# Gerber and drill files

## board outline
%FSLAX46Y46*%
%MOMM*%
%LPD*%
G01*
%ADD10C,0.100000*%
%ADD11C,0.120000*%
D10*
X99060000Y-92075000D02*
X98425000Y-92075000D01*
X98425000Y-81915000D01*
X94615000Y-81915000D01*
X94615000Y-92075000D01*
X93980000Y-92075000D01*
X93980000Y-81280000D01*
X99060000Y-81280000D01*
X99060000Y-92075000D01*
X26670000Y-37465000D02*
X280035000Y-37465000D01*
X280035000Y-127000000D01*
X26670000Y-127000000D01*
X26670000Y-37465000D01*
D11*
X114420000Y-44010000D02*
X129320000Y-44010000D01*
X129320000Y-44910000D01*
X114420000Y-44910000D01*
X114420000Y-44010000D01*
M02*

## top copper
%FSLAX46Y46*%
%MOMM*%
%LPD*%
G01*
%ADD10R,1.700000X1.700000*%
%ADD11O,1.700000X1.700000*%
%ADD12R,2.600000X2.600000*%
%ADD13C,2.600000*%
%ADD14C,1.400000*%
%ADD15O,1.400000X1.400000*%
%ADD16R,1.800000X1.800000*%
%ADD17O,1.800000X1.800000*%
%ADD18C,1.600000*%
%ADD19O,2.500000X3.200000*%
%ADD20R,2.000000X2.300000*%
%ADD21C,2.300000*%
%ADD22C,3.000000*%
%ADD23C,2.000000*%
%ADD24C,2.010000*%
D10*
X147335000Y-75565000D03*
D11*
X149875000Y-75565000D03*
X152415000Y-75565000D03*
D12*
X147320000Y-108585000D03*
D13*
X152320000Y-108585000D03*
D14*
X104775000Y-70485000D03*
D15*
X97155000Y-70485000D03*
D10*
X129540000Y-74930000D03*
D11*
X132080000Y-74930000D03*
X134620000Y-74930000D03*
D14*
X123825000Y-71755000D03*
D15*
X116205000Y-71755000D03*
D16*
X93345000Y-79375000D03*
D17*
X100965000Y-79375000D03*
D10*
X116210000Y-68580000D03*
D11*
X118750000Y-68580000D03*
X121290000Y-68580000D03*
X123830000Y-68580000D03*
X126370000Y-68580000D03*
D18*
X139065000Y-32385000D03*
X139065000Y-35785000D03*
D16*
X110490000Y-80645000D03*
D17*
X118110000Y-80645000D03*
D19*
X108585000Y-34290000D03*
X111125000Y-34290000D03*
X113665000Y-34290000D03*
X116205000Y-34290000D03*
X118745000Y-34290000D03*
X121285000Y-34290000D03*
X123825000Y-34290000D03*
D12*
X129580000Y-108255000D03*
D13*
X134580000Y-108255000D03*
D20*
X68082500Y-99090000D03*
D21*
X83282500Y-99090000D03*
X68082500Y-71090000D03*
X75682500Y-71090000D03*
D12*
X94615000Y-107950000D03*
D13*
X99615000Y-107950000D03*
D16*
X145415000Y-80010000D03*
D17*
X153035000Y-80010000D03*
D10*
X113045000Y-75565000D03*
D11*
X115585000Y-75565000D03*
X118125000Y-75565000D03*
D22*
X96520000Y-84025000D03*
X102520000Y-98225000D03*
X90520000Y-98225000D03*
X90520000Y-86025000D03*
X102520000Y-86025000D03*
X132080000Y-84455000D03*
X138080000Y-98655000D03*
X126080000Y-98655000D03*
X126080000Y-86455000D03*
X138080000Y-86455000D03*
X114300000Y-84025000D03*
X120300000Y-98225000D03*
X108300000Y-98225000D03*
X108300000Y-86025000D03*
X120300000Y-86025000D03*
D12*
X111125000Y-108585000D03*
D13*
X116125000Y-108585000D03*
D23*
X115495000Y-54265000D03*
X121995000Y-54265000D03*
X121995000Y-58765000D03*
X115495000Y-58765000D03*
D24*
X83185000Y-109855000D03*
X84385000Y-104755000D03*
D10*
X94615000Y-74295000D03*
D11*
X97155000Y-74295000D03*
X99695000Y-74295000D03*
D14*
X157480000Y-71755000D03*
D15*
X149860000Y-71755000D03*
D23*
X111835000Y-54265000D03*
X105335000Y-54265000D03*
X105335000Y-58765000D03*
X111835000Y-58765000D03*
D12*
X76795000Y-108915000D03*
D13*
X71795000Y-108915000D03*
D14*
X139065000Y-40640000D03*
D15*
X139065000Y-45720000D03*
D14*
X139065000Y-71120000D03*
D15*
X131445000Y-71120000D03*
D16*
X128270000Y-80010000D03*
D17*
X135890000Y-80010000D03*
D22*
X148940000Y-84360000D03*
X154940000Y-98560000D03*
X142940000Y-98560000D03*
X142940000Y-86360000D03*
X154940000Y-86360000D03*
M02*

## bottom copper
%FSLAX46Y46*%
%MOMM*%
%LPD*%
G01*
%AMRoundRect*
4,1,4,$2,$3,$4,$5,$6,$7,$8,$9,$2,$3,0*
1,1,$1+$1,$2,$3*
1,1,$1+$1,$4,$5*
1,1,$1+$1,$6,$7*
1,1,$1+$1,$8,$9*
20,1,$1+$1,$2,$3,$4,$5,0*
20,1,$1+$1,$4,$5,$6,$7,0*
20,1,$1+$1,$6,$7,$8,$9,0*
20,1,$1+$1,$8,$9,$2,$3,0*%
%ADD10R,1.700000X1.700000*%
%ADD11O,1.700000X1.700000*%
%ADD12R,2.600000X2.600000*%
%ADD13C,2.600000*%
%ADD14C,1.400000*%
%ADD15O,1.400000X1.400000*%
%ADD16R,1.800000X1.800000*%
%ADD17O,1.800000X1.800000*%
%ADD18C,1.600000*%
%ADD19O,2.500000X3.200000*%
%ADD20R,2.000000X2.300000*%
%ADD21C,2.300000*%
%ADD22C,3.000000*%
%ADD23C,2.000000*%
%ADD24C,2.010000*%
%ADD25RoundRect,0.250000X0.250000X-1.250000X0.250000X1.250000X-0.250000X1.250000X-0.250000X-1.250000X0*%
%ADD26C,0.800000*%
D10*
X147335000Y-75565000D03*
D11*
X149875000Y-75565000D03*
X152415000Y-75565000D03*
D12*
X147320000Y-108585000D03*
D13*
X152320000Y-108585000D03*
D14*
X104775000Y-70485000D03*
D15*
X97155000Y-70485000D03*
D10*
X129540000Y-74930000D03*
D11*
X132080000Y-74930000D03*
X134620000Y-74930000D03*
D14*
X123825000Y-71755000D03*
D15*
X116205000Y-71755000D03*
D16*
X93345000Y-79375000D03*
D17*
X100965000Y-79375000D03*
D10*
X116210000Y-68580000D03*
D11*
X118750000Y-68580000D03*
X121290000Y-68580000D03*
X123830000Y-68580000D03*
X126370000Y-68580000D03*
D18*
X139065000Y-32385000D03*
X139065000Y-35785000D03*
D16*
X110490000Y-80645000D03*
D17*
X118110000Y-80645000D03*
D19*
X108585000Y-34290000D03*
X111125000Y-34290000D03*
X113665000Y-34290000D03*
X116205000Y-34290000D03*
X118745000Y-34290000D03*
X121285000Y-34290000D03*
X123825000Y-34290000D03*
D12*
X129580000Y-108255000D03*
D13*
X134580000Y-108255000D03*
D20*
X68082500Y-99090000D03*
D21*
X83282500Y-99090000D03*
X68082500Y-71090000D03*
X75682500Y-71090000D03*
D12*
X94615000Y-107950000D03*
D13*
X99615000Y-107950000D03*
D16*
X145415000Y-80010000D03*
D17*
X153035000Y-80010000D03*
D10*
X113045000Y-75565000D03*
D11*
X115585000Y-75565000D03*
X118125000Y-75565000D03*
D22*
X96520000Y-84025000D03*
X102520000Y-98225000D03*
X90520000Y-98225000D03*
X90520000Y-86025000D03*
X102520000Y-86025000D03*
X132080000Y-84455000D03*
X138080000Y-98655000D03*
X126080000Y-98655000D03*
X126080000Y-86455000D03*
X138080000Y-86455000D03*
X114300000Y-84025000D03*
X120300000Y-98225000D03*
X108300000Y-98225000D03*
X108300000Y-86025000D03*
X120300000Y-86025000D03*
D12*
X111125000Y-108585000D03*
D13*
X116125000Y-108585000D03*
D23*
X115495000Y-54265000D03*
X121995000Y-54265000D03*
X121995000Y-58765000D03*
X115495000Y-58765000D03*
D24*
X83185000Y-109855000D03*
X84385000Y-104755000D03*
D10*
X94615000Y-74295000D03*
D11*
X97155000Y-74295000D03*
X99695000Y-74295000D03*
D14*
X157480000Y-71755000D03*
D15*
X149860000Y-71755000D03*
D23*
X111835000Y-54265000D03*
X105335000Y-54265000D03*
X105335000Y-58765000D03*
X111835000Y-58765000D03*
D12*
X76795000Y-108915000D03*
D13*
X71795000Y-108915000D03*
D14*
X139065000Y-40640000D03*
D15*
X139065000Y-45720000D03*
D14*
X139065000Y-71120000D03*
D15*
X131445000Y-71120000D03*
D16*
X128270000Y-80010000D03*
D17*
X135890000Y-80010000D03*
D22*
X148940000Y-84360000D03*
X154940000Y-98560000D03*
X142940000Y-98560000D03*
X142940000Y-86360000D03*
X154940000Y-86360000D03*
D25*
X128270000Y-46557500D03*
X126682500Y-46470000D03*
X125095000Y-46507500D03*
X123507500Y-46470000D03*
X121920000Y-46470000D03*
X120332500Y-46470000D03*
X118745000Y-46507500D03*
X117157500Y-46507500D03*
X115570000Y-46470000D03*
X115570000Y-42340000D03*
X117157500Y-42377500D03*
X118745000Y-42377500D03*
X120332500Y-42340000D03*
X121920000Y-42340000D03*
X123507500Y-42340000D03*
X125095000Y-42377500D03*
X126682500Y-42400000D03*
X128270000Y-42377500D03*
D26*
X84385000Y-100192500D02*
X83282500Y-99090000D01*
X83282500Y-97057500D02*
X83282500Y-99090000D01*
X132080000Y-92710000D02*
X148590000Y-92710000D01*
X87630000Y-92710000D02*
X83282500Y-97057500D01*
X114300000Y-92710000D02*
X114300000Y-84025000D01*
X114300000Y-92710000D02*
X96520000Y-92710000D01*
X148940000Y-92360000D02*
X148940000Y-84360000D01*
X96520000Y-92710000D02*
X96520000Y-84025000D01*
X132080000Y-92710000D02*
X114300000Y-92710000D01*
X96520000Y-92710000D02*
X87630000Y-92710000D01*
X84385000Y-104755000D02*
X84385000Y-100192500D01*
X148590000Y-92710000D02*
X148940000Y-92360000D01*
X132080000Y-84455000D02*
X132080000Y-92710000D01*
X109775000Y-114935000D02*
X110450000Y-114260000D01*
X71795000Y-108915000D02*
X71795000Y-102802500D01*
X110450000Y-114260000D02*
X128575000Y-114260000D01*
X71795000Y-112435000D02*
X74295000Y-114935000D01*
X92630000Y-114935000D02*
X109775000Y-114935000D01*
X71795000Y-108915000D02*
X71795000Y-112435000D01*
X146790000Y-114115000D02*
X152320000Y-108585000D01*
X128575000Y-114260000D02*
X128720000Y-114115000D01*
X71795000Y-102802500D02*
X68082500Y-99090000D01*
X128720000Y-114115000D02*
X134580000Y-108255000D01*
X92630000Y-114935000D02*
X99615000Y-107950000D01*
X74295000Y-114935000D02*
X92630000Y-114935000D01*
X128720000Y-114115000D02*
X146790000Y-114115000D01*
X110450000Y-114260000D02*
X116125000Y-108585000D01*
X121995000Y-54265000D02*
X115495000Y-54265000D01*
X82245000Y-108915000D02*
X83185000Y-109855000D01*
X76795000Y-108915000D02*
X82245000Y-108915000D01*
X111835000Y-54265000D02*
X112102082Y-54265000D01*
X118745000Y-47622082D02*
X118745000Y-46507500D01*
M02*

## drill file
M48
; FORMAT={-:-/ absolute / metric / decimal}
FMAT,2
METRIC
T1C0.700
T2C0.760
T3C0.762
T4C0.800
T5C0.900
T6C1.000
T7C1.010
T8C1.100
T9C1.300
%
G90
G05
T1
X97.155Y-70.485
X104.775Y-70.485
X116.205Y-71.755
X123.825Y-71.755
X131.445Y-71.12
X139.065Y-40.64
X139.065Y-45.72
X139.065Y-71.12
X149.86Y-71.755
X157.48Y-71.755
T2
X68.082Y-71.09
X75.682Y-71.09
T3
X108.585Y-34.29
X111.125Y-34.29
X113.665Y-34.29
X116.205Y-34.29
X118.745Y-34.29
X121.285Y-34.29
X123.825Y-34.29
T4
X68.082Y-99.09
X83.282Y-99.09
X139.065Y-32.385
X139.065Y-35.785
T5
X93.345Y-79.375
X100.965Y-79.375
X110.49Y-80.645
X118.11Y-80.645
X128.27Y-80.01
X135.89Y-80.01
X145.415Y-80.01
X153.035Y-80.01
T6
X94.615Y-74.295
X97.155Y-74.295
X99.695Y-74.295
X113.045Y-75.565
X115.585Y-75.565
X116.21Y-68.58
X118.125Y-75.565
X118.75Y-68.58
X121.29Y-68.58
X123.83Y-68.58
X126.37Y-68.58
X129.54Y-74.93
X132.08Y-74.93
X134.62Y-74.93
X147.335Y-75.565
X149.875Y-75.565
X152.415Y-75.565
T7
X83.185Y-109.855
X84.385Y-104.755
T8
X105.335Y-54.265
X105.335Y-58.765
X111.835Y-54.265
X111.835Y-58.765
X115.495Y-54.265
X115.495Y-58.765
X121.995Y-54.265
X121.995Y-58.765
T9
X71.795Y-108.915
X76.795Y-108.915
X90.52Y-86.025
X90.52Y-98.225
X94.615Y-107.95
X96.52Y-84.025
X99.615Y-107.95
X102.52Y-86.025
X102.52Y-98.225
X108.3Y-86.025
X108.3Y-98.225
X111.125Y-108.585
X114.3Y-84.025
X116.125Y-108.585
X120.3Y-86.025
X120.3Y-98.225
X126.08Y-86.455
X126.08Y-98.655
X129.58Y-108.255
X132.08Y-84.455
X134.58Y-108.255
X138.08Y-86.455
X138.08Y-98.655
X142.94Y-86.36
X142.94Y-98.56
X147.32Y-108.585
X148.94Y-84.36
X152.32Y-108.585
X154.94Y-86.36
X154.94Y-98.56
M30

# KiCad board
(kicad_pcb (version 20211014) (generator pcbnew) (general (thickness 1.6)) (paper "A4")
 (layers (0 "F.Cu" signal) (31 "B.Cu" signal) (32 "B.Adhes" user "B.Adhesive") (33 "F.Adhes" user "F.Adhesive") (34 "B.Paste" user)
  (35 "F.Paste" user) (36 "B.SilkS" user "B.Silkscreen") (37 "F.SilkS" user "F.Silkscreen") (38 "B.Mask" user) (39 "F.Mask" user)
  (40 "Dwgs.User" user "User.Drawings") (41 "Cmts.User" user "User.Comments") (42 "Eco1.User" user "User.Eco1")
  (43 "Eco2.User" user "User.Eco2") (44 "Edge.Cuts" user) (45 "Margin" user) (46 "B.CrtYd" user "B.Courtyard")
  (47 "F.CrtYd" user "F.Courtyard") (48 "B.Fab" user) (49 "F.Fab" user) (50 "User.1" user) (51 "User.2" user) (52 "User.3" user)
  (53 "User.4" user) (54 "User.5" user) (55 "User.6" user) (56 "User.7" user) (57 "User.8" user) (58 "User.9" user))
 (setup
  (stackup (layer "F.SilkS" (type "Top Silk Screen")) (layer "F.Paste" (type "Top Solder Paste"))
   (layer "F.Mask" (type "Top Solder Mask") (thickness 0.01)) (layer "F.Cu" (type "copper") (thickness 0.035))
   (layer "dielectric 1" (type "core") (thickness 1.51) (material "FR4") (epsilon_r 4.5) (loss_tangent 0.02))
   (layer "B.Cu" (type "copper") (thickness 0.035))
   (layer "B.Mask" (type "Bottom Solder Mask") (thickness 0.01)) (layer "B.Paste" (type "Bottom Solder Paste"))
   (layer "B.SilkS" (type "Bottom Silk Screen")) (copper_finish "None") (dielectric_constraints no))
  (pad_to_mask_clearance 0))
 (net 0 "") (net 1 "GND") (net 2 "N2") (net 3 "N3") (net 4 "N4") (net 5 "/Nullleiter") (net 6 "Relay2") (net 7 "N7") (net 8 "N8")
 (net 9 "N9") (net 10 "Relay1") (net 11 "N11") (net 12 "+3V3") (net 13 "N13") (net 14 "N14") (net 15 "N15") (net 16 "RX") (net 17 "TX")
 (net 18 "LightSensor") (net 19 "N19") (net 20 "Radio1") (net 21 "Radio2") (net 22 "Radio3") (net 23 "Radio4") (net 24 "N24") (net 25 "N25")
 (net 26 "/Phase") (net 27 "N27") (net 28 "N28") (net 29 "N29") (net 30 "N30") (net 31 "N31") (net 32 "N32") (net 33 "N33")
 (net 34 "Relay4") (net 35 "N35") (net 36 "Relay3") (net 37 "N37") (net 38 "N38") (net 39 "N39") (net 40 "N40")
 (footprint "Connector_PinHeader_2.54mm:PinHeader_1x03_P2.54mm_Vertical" (layer "F.Cu") (at 147.335 75.565 90)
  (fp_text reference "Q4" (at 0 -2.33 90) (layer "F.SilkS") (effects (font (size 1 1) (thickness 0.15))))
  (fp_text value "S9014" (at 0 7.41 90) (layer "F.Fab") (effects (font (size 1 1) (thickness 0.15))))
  (pad "1" thru_hole rect (at 0 0 90) (size 1.7 1.7) (drill 1) (layers *.Cu *.Mask) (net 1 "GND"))
  (pad "2" thru_hole oval (at 0 2.54 90) (size 1.7 1.7) (drill 1) (layers *.Cu *.Mask) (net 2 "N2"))
  (pad "3" thru_hole oval (at 0 5.08 90) (size 1.7 1.7) (drill 1) (layers *.Cu *.Mask) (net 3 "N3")))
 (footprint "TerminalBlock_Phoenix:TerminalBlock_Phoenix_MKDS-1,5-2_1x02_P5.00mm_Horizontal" (layer "F.Cu") (at 147.32 108.585)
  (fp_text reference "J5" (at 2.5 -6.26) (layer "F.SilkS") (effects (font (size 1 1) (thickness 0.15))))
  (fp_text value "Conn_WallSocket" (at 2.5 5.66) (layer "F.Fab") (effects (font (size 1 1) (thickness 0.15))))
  (pad "1" thru_hole rect (at 0 0) (size 2.6 2.6) (drill 1.3) (layers *.Cu *.Mask) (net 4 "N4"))
  (pad "2" thru_hole circle (at 5 0) (size 2.6 2.6) (drill 1.3) (layers *.Cu *.Mask) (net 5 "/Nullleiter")))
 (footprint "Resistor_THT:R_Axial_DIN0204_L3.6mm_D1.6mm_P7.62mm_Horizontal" (layer "F.Cu") (at 104.775 70.485 180)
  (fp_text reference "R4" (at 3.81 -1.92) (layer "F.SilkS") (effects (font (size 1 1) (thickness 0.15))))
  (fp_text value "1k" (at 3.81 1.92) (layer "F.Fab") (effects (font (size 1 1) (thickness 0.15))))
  (pad "1" thru_hole circle (at 0 0 180) (size 1.4 1.4) (drill 0.7) (layers *.Cu *.Mask) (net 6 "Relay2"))
  (pad "2" thru_hole oval (at 7.62 0 180) (size 1.4 1.4) (drill 0.7) (layers *.Cu *.Mask) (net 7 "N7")))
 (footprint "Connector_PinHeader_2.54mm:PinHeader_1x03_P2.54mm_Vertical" (layer "F.Cu") (at 129.54 74.93 90)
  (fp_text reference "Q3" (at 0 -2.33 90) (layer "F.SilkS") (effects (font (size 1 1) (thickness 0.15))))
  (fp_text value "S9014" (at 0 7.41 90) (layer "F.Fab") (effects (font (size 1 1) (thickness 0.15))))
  (pad "1" thru_hole rect (at 0 0 90) (size 1.7 1.7) (drill 1) (layers *.Cu *.Mask) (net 1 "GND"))
  (pad "2" thru_hole oval (at 0 2.54 90) (size 1.7 1.7) (drill 1) (layers *.Cu *.Mask) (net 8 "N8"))
  (pad "3" thru_hole oval (at 0 5.08 90) (size 1.7 1.7) (drill 1) (layers *.Cu *.Mask) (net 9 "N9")))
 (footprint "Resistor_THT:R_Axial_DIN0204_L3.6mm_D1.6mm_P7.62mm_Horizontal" (layer "F.Cu") (at 123.825 71.755 180)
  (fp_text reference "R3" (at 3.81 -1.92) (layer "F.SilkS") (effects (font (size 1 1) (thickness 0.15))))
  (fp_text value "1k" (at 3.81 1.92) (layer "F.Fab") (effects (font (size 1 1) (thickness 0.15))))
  (pad "1" thru_hole circle (at 0 0 180) (size 1.4 1.4) (drill 0.7) (layers *.Cu *.Mask) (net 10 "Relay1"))
  (pad "2" thru_hole oval (at 7.62 0 180) (size 1.4 1.4) (drill 0.7) (layers *.Cu *.Mask) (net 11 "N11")))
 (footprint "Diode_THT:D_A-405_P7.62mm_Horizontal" (layer "F.Cu") (at 93.345 79.375)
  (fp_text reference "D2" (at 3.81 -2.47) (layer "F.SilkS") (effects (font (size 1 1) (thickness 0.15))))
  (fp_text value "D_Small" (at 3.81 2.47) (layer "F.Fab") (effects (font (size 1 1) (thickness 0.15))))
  (pad "1" thru_hole rect (at 0 0) (size 1.8 1.8) (drill 0.9) (layers *.Cu *.Mask) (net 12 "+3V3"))
  (pad "2" thru_hole oval (at 7.62 0) (size 1.8 1.8) (drill 0.9) (layers *.Cu *.Mask) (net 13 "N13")))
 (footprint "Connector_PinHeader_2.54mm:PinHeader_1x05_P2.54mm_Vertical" (layer "F.Cu") (at 116.21 68.58 90)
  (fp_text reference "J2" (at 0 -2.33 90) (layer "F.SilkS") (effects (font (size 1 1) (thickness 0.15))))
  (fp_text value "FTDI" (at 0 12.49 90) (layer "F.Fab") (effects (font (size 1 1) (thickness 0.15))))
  (pad "1" thru_hole rect (at 0 0 90) (size 1.7 1.7) (drill 1) (layers *.Cu *.Mask) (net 1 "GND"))
  (pad "2" thru_hole oval (at 0 2.54 90) (size 1.7 1.7) (drill 1) (layers *.Cu *.Mask) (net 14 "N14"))
  (pad "3" thru_hole oval (at 0 5.08 90) (size 1.7 1.7) (drill 1) (layers *.Cu *.Mask) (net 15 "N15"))
  (pad "4" thru_hole oval (at 0 7.62 90) (size 1.7 1.7) (drill 1) (layers *.Cu *.Mask) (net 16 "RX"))
  (pad "5" thru_hole oval (at 0 10.16 90) (size 1.7 1.7) (drill 1) (layers *.Cu *.Mask) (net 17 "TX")))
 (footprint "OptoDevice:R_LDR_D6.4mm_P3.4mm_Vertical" (layer "F.Cu") (at 139.065 32.385 -90)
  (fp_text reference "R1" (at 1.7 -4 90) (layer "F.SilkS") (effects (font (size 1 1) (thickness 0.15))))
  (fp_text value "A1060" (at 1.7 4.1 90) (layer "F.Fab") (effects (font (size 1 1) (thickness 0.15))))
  (pad "1" thru_hole circle (at 0 0 270) (size 1.6 1.6) (drill 0.8) (layers *.Cu *.Mask) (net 12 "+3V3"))
  (pad "2" thru_hole circle (at 3.4 0 270) (size 1.6 1.6) (drill 0.8) (layers *.Cu *.Mask) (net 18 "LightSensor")))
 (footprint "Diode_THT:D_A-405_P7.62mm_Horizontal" (layer "F.Cu") (at 110.49 80.645)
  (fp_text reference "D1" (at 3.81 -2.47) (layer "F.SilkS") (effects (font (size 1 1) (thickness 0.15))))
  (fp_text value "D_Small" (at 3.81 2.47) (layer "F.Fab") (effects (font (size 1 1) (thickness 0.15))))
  (pad "1" thru_hole rect (at 0 0) (size 1.8 1.8) (drill 0.9) (layers *.Cu *.Mask) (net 12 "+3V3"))
  (pad "2" thru_hole oval (at 7.62 0) (size 1.8 1.8) (drill 0.9) (layers *.Cu *.Mask) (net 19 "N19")))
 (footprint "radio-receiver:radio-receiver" (layer "F.Cu") (at 108.585 34.29)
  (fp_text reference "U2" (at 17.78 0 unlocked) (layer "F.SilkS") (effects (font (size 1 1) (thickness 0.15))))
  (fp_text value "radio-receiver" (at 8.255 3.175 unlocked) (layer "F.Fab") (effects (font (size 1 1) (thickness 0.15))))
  (pad "1" thru_hole oval (at 0 0 270) (size 3.2 2.5) (drill 0.762) (layers *.Cu *.Mask) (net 1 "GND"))
  (pad "2" thru_hole oval (at 2.54 0 270) (size 3.2 2.5) (drill 0.762) (layers *.Cu *.Mask) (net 12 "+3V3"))
  (pad "3" thru_hole oval (at 5.08 0 270) (size 3.2 2.5) (drill 0.762) (layers *.Cu *.Mask) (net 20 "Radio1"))
  (pad "4" thru_hole oval (at 7.62 0 270) (size 3.2 2.5) (drill 0.762) (layers *.Cu *.Mask) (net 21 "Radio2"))
  (pad "5" thru_hole oval (at 10.16 0 270) (size 3.2 2.5) (drill 0.762) (layers *.Cu *.Mask) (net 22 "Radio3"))
  (pad "6" thru_hole oval (at 12.7 0 270) (size 3.2 2.5) (drill 0.762) (layers *.Cu *.Mask) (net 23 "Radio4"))
  (pad "7" thru_hole oval (at 15.24 0 270) (size 3.2 2.5) (drill 0.762) (layers *.Cu *.Mask) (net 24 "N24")))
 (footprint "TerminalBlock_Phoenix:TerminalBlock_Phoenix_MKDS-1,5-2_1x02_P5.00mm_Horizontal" (layer "F.Cu") (at 129.58 108.255)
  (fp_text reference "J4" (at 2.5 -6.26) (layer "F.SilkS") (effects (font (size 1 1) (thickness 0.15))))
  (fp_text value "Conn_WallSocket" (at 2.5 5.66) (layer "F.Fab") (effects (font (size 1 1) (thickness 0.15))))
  (pad "1" thru_hole rect (at 0 0) (size 2.6 2.6) (drill 1.3) (layers *.Cu *.Mask) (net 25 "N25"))
  (pad "2" thru_hole circle (at 5 0) (size 2.6 2.6) (drill 1.3) (layers *.Cu *.Mask) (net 5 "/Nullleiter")))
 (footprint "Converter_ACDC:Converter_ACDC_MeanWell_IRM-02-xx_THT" (layer "F.Cu") (at 68.0825 99.09 90)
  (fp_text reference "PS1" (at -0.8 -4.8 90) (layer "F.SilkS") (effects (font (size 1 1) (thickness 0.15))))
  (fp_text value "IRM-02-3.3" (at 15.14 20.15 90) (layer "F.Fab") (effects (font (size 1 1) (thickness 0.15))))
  (pad "1" thru_hole rect (at 0 0 90) (size 2.3 2) (drill 0.8) (layers *.Cu *.Mask) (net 5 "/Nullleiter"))
  (pad "2" thru_hole circle (at 0 15.2 90) (size 2.3 2.3) (drill 0.8) (layers *.Cu *.Mask) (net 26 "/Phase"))
  (pad "3" thru_hole circle (at 28 0 90) (size 2.3 2.3) (drill 0.76) (layers *.Cu *.Mask) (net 1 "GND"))
  (pad "4" thru_hole circle (at 28 7.6 90) (size 2.3 2.3) (drill 0.76) (layers *.Cu *.Mask) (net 12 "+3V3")))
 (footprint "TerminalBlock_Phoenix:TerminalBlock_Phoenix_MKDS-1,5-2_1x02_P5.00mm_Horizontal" (layer "F.Cu") (at 94.615 107.95)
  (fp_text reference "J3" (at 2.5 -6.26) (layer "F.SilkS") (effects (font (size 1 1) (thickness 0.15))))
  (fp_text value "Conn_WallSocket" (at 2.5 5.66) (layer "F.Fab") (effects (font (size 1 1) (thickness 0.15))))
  (pad "1" thru_hole rect (at 0 0) (size 2.6 2.6) (drill 1.3) (layers *.Cu *.Mask) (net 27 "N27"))
  (pad "2" thru_hole circle (at 5 0) (size 2.6 2.6) (drill 1.3) (layers *.Cu *.Mask) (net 5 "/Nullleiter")))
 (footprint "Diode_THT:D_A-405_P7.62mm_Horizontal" (layer "F.Cu") (at 145.415 80.01)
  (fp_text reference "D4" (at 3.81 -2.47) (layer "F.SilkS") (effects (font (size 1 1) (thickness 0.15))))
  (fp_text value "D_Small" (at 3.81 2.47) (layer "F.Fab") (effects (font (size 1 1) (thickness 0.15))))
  (pad "1" thru_hole rect (at 0 0) (size 1.8 1.8) (drill 0.9) (layers *.Cu *.Mask) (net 12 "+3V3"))
  (pad "2" thru_hole oval (at 7.62 0) (size 1.8 1.8) (drill 0.9) (layers *.Cu *.Mask) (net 3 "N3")))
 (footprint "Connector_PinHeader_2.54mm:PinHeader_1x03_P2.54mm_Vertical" (layer "F.Cu") (at 113.045 75.565 90)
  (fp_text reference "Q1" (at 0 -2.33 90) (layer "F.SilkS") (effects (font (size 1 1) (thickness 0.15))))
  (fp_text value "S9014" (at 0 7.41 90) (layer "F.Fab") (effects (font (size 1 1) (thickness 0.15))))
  (pad "1" thru_hole rect (at 0 0 90) (size 1.7 1.7) (drill 1) (layers *.Cu *.Mask) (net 1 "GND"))
  (pad "2" thru_hole oval (at 0 2.54 90) (size 1.7 1.7) (drill 1) (layers *.Cu *.Mask) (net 11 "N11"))
  (pad "3" thru_hole oval (at 0 5.08 90) (size 1.7 1.7) (drill 1) (layers *.Cu *.Mask) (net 19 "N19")))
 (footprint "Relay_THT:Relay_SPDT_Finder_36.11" (layer "F.Cu") (at 96.52 84.025 -90)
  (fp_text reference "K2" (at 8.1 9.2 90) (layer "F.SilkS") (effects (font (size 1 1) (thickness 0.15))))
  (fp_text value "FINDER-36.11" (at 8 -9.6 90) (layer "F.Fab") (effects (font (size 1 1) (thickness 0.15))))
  (pad "11" thru_hole circle (at 0 0 270) (size 3 3) (drill 1.3) (layers *.Cu *.Mask) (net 26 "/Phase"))
  (pad "12" thru_hole circle (at 14.2 -6 270) (size 3 3) (drill 1.3) (layers *.Cu *.Mask) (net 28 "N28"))
  (pad "14" thru_hole circle (at 14.2 6 270) (size 3 3) (drill 1.3) (layers *.Cu *.Mask) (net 27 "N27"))
  (pad "A1" thru_hole circle (at 2 6 270) (size 3 3) (drill 1.3) (layers *.Cu *.Mask) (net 12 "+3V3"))
  (pad "A2" thru_hole circle (at 2 -6 270) (size 3 3) (drill 1.3) (layers *.Cu *.Mask) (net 13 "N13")))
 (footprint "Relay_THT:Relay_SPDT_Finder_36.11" (layer "F.Cu") (at 132.08 84.455 -90)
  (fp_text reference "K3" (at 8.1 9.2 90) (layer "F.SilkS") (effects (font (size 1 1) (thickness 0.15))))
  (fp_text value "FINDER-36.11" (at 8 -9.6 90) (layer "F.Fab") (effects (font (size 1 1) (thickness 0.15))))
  (pad "11" thru_hole circle (at 0 0 270) (size 3 3) (drill 1.3) (layers *.Cu *.Mask) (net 26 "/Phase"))
  (pad "12" thru_hole circle (at 14.2 -6 270) (size 3 3) (drill 1.3) (layers *.Cu *.Mask) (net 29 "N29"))
  (pad "14" thru_hole circle (at 14.2 6 270) (size 3 3) (drill 1.3) (layers *.Cu *.Mask) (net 25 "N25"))
  (pad "A1" thru_hole circle (at 2 6 270) (size 3 3) (drill 1.3) (layers *.Cu *.Mask) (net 12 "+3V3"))
  (pad "A2" thru_hole circle (at 2 -6 270) (size 3 3) (drill 1.3) (layers *.Cu *.Mask) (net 9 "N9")))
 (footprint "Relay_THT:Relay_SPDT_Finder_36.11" (layer "F.Cu") (at 114.3 84.025 -90)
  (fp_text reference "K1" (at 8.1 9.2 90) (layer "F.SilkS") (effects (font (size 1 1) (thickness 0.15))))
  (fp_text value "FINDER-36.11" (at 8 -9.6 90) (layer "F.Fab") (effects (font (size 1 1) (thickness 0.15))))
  (pad "11" thru_hole circle (at 0 0 270) (size 3 3) (drill 1.3) (layers *.Cu *.Mask) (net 26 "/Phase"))
  (pad "12" thru_hole circle (at 14.2 -6 270) (size 3 3) (drill 1.3) (layers *.Cu *.Mask) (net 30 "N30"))
  (pad "14" thru_hole circle (at 14.2 6 270) (size 3 3) (drill 1.3) (layers *.Cu *.Mask) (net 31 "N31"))
  (pad "A1" thru_hole circle (at 2 6 270) (size 3 3) (drill 1.3) (layers *.Cu *.Mask) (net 12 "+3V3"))
  (pad "A2" thru_hole circle (at 2 -6 270) (size 3 3) (drill 1.3) (layers *.Cu *.Mask) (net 19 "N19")))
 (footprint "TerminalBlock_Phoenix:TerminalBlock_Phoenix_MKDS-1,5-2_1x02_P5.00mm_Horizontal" (layer "F.Cu") (at 111.125 108.585)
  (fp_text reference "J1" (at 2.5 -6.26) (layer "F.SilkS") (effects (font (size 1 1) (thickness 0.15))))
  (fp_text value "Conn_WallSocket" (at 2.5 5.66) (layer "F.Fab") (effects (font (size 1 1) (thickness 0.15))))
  (pad "1" thru_hole rect (at 0 0) (size 2.6 2.6) (drill 1.3) (layers *.Cu *.Mask) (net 31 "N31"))
  (pad "2" thru_hole circle (at 5 0) (size 2.6 2.6) (drill 1.3) (layers *.Cu *.Mask) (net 5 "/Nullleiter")))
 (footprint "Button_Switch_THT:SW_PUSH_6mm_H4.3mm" (layer "F.Cu") (at 115.495 54.265)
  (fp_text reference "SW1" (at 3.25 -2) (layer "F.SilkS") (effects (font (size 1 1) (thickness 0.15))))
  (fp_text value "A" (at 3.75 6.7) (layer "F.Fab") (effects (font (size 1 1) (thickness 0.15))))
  (pad "1" thru_hole circle (at 0 0 90) (size 2 2) (drill 1.1) (layers *.Cu *.Mask) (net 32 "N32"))
  (pad "1" thru_hole circle (at 6.5 0 90) (size 2 2) (drill 1.1) (layers *.Cu *.Mask) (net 32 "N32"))
  (pad "2" thru_hole circle (at 6.5 4.5 90) (size 2 2) (drill 1.1) (layers *.Cu *.Mask) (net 1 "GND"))
  (pad "2" thru_hole circle (at 0 4.5 90) (size 2 2) (drill 1.1) (layers *.Cu *.Mask) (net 1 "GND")))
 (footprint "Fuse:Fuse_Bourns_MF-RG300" (layer "F.Cu") (at 83.185 109.855 90)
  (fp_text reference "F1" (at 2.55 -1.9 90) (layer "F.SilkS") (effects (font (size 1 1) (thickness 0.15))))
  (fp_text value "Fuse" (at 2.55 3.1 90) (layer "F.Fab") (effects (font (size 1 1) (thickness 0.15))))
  (pad "1" thru_hole circle (at 0 0 90) (size 2.01 2.01) (drill 1.01) (layers *.Cu *.Mask) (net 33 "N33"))
  (pad "2" thru_hole circle (at 5.1 1.2 90) (size 2.01 2.01) (drill 1.01) (layers *.Cu *.Mask) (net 26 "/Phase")))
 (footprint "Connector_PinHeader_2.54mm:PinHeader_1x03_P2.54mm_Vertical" (layer "F.Cu") (at 94.615 74.295 90)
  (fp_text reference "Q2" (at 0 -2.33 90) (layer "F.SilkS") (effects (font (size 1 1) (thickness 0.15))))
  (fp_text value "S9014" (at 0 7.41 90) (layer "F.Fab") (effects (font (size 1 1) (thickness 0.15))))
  (pad "1" thru_hole rect (at 0 0 90) (size 1.7 1.7) (drill 1) (layers *.Cu *.Mask) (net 1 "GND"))
  (pad "2" thru_hole oval (at 0 2.54 90) (size 1.7 1.7) (drill 1) (layers *.Cu *.Mask) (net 7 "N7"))
  (pad "3" thru_hole oval (at 0 5.08 90) (size 1.7 1.7) (drill 1) (layers *.Cu *.Mask) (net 13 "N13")))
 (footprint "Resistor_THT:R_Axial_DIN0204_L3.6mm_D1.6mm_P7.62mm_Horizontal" (layer "F.Cu") (at 157.48 71.755 180)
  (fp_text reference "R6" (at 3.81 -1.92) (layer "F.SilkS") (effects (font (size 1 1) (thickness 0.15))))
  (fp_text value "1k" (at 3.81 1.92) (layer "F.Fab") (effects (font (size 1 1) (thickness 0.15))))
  (pad "1" thru_hole circle (at 0 0 180) (size 1.4 1.4) (drill 0.7) (layers *.Cu *.Mask) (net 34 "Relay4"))
  (pad "2" thru_hole oval (at 7.62 0 180) (size 1.4 1.4) (drill 0.7) (layers *.Cu *.Mask) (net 2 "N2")))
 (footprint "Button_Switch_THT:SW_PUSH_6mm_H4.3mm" (layer "F.Cu") (at 105.335 54.265)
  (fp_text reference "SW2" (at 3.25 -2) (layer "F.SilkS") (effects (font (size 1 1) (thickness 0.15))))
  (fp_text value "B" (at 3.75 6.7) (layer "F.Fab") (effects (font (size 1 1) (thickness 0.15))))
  (pad "1" thru_hole circle (at 6.5 0 90) (size 2 2) (drill 1.1) (layers *.Cu *.Mask) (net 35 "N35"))
  (pad "1" thru_hole circle (at 0 0 90) (size 2 2) (drill 1.1) (layers *.Cu *.Mask) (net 35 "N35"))
  (pad "2" thru_hole circle (at 0 4.5 90) (size 2 2) (drill 1.1) (layers *.Cu *.Mask) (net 1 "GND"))
  (pad "2" thru_hole circle (at 6.5 4.5 90) (size 2 2) (drill 1.1) (layers *.Cu *.Mask) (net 1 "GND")))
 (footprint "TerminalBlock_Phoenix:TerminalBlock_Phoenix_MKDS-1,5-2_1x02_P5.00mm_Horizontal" (layer "F.Cu") (at 76.795 108.915 180)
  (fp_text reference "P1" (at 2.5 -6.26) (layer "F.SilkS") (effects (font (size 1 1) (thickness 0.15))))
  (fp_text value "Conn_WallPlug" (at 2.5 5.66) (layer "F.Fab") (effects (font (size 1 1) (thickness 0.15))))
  (pad "1" thru_hole rect (at 0 0 180) (size 2.6 2.6) (drill 1.3) (layers *.Cu *.Mask) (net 33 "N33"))
  (pad "2" thru_hole circle (at 5 0 180) (size 2.6 2.6) (drill 1.3) (layers *.Cu *.Mask) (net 5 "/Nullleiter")))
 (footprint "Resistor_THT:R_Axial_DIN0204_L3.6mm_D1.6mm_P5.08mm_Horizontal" (layer "F.Cu") (at 139.065 40.64 -90)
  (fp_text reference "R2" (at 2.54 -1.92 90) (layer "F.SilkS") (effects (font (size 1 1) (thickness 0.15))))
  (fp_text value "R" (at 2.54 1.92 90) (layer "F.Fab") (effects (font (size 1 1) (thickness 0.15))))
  (pad "1" thru_hole circle (at 0 0 270) (size 1.4 1.4) (drill 0.7) (layers *.Cu *.Mask) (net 18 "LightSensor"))
  (pad "2" thru_hole oval (at 5.08 0 270) (size 1.4 1.4) (drill 0.7) (layers *.Cu *.Mask) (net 1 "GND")))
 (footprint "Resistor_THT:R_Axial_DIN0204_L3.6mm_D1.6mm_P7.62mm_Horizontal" (layer "F.Cu") (at 139.065 71.12 180)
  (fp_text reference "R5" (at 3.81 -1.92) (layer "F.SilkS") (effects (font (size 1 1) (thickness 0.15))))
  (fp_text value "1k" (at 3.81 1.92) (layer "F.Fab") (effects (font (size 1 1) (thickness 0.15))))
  (pad "1" thru_hole circle (at 0 0 180) (size 1.4 1.4) (drill 0.7) (layers *.Cu *.Mask) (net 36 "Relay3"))
  (pad "2" thru_hole oval (at 7.62 0 180) (size 1.4 1.4) (drill 0.7) (layers *.Cu *.Mask) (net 8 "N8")))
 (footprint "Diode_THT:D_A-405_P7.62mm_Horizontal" (layer "F.Cu") (at 128.27 80.01)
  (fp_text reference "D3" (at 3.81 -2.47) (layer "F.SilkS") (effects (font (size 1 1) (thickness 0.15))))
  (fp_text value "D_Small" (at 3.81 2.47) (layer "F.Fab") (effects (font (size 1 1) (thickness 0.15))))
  (pad "1" thru_hole rect (at 0 0) (size 1.8 1.8) (drill 0.9) (layers *.Cu *.Mask) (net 12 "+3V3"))
  (pad "2" thru_hole oval (at 7.62 0) (size 1.8 1.8) (drill 0.9) (layers *.Cu *.Mask) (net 9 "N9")))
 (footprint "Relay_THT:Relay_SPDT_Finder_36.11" (layer "F.Cu") (at 148.94 84.36 -90)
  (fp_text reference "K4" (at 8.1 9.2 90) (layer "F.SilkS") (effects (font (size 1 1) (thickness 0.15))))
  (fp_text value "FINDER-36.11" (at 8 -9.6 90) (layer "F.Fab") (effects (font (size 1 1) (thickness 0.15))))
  (pad "11" thru_hole circle (at 0 0 270) (size 3 3) (drill 1.3) (layers *.Cu *.Mask) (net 26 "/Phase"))
  (pad "12" thru_hole circle (at 14.2 -6 270) (size 3 3) (drill 1.3) (layers *.Cu *.Mask) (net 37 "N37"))
  (pad "14" thru_hole circle (at 14.2 6 270) (size 3 3) (drill 1.3) (layers *.Cu *.Mask) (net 4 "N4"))
  (pad "A1" thru_hole circle (at 2 6 270) (size 3 3) (drill 1.3) (layers *.Cu *.Mask) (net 12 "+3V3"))
  (pad "A2" thru_hole circle (at 2 -6 270) (size 3 3) (drill 1.3) (layers *.Cu *.Mask) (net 3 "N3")))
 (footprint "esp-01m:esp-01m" (layer "B.Cu") (at 121.92 44.45 90)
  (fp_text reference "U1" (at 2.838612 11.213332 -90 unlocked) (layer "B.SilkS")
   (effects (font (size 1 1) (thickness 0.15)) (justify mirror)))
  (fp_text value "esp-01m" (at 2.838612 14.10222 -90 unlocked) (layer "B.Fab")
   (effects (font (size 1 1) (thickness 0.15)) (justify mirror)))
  (fp_rect (start -0.46 7.4) (end 0.44 -7.5) (layer "Edge.Cuts") (width 0.12) (fill none))
  (pad "1" smd roundrect (at -2.1075 6.35 90) (size 3 1) (layers "B.Cu" "B.Paste" "B.Mask") (roundrect_rratio 0.25) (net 1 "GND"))
  (pad "2" smd roundrect (at -2.02 4.7625 90) (size 3 1) (layers "B.Cu" "B.Paste" "B.Mask") (roundrect_rratio 0.25) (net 12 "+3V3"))
  (pad "3" smd roundrect (at -2.0575 3.175 90) (size 3 1) (layers "B.Cu" "B.Paste" "B.Mask") (roundrect_rratio 0.25) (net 17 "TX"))
  (pad "4" smd roundrect (at -2.02 1.5875 90) (size 3 1) (layers "B.Cu" "B.Paste" "B.Mask") (roundrect_rratio 0.25) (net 16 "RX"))
  (pad "5" smd roundrect (at -2.02 0 90) (size 3 1) (layers "B.Cu" "B.Paste" "B.Mask") (roundrect_rratio 0.25) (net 32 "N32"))
  (pad "6" smd roundrect (at -2.02 -1.5875 90) (size 3 1) (layers "B.Cu" "B.Paste" "B.Mask") (roundrect_rratio 0.25) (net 34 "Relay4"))
  (pad "7" smd roundrect (at -2.0575 -3.175 90) (size 3 1) (layers "B.Cu" "B.Paste" "B.Mask") (roundrect_rratio 0.25) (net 35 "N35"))
  (pad "8" smd roundrect (at -2.0575 -4.7625 90) (size 3 1) (layers "B.Cu" "B.Paste" "B.Mask") (roundrect_rratio 0.25) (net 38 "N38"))
  (pad "9" smd roundrect (at -2.02 -6.35 90) (size 3 1) (layers "B.Cu" "B.Paste" "B.Mask") (roundrect_rratio 0.25) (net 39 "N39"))
  (pad "10" smd roundrect (at 2.11 -6.35 90) (size 3 1) (layers "B.Cu" "B.Paste" "B.Mask") (roundrect_rratio 0.25) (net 20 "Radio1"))
  (pad "11" smd roundrect (at 2.0725 -4.7625 90) (size 3 1) (layers "B.Cu" "B.Paste" "B.Mask") (roundrect_rratio 0.25) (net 21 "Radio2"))
  (pad "12" smd roundrect (at 2.0725 -3.175 90) (size 3 1) (layers "B.Cu" "B.Paste" "B.Mask") (roundrect_rratio 0.25) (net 22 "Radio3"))
  (pad "13" smd roundrect (at 2.11 -1.5875 90) (size 3 1) (layers "B.Cu" "B.Paste" "B.Mask") (roundrect_rratio 0.25) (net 23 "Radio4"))
  (pad "14" smd roundrect (at 2.11 0 90) (size 3 1) (layers "B.Cu" "B.Paste" "B.Mask") (roundrect_rratio 0.25) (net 10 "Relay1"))
  (pad "15" smd roundrect (at 2.11 1.5875 90) (size 3 1) (layers "B.Cu" "B.Paste" "B.Mask") (roundrect_rratio 0.25) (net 6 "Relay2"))
  (pad "16" smd roundrect (at 2.0725 3.175 90) (size 3 1) (layers "B.Cu" "B.Paste" "B.Mask") (roundrect_rratio 0.25) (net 18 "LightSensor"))
  (pad "17" smd roundrect (at 2.05 4.7625 90) (size 3 1) (layers "B.Cu" "B.Paste" "B.Mask") (roundrect_rratio 0.25) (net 36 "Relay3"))
  (pad "18" smd roundrect (at 2.0725 6.35 90) (size 3 1) (layers "B.Cu" "B.Paste" "B.Mask") (roundrect_rratio 0.25) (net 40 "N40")))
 (gr_poly
  (pts (xy 99.06 92.075) (xy 98.425 92.075) (xy 98.425 81.915) (xy 94.615 81.915) (xy 94.615 92.075) (xy 93.98 92.075) (xy 93.98 81.28)
   (xy 99.06 81.28))
  (layer "Edge.Cuts") (width 0.1) (fill none))
 (gr_rect (start 26.67 37.465) (end 280.035 127) (layer "Edge.Cuts") (width 0.1) (fill none))
 (segment (start 84.385 100.1925) (end 83.2825 99.09) (width 0.8) (layer "B.Cu") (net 26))
 (segment (start 83.2825 97.0575) (end 83.2825 99.09) (width 0.8) (layer "B.Cu") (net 26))
 (segment (start 132.08 92.71) (end 148.59 92.71) (width 0.8) (layer "B.Cu") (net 26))
 (segment (start 87.63 92.71) (end 83.2825 97.0575) (width 0.8) (layer "B.Cu") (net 26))
 (segment (start 114.3 92.71) (end 114.3 84.025) (width 0.8) (layer "B.Cu") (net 26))
 (segment (start 114.3 92.71) (end 96.52 92.71) (width 0.8) (layer "B.Cu") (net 26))
 (segment (start 148.94 92.36) (end 148.94 84.36) (width 0.8) (layer "B.Cu") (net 26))
 (segment (start 96.52 92.71) (end 96.52 84.025) (width 0.8) (layer "B.Cu") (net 26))
 (segment (start 132.08 92.71) (end 114.3 92.71) (width 0.8) (layer "B.Cu") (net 26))
 (segment (start 96.52 92.71) (end 87.63 92.71) (width 0.8) (layer "B.Cu") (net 26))
 (segment (start 84.385 104.755) (end 84.385 100.1925) (width 0.8) (layer "B.Cu") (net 26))
 (segment (start 148.59 92.71) (end 148.94 92.36) (width 0.8) (layer "B.Cu") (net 26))
 (segment (start 132.08 84.455) (end 132.08 92.71) (width 0.8) (layer "B.Cu") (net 26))
 (segment (start 109.775 114.935) (end 110.45 114.26) (width 0.8) (layer "B.Cu") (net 5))
 (segment (start 71.795 108.915) (end 71.795 102.8025) (width 0.8) (layer "B.Cu") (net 5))
 (segment (start 110.45 114.26) (end 128.575 114.26) (width 0.8) (layer "B.Cu") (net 5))
 (segment (start 71.795 112.435) (end 74.295 114.935) (width 0.8) (layer "B.Cu") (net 5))
 (segment (start 92.63 114.935) (end 109.775 114.935) (width 0.8) (layer "B.Cu") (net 5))
 (segment (start 71.795 108.915) (end 71.795 112.435) (width 0.8) (layer "B.Cu") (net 5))
 (segment (start 146.79 114.115) (end 152.32 108.585) (width 0.8) (layer "B.Cu") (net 5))
 (segment (start 128.575 114.26) (end 128.72 114.115) (width 0.8) (layer "B.Cu") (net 5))
 (segment (start 71.795 102.8025) (end 68.0825 99.09) (width 0.8) (layer "B.Cu") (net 5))
 (segment (start 128.72 114.115) (end 134.58 108.255) (width 0.8) (layer "B.Cu") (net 5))
 (segment (start 92.63 114.935) (end 99.615 107.95) (width 0.8) (layer "B.Cu") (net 5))
 (segment (start 74.295 114.935) (end 92.63 114.935) (width 0.8) (layer "B.Cu") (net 5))
 (segment (start 128.72 114.115) (end 146.79 114.115) (width 0.8) (layer "B.Cu") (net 5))
 (segment (start 110.45 114.26) (end 116.125 108.585) (width 0.8) (layer "B.Cu") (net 5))
 (segment (start 121.995 54.265) (end 115.495 54.265) (width 0.8) (layer "B.Cu") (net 32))
 (segment (start 82.245 108.915) (end 83.185 109.855) (width 0.8) (layer "B.Cu") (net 33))
 (segment (start 76.795 108.915) (end 82.245 108.915) (width 0.8) (layer "B.Cu") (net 33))
 (segment (start 111.835 54.265) (end 112.102082 54.265) (width 0.8) (layer "B.Cu") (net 35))
 (segment (start 118.745 47.622082) (end 118.745 46.5075) (width 0.8) (layer "B.Cu") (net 35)))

